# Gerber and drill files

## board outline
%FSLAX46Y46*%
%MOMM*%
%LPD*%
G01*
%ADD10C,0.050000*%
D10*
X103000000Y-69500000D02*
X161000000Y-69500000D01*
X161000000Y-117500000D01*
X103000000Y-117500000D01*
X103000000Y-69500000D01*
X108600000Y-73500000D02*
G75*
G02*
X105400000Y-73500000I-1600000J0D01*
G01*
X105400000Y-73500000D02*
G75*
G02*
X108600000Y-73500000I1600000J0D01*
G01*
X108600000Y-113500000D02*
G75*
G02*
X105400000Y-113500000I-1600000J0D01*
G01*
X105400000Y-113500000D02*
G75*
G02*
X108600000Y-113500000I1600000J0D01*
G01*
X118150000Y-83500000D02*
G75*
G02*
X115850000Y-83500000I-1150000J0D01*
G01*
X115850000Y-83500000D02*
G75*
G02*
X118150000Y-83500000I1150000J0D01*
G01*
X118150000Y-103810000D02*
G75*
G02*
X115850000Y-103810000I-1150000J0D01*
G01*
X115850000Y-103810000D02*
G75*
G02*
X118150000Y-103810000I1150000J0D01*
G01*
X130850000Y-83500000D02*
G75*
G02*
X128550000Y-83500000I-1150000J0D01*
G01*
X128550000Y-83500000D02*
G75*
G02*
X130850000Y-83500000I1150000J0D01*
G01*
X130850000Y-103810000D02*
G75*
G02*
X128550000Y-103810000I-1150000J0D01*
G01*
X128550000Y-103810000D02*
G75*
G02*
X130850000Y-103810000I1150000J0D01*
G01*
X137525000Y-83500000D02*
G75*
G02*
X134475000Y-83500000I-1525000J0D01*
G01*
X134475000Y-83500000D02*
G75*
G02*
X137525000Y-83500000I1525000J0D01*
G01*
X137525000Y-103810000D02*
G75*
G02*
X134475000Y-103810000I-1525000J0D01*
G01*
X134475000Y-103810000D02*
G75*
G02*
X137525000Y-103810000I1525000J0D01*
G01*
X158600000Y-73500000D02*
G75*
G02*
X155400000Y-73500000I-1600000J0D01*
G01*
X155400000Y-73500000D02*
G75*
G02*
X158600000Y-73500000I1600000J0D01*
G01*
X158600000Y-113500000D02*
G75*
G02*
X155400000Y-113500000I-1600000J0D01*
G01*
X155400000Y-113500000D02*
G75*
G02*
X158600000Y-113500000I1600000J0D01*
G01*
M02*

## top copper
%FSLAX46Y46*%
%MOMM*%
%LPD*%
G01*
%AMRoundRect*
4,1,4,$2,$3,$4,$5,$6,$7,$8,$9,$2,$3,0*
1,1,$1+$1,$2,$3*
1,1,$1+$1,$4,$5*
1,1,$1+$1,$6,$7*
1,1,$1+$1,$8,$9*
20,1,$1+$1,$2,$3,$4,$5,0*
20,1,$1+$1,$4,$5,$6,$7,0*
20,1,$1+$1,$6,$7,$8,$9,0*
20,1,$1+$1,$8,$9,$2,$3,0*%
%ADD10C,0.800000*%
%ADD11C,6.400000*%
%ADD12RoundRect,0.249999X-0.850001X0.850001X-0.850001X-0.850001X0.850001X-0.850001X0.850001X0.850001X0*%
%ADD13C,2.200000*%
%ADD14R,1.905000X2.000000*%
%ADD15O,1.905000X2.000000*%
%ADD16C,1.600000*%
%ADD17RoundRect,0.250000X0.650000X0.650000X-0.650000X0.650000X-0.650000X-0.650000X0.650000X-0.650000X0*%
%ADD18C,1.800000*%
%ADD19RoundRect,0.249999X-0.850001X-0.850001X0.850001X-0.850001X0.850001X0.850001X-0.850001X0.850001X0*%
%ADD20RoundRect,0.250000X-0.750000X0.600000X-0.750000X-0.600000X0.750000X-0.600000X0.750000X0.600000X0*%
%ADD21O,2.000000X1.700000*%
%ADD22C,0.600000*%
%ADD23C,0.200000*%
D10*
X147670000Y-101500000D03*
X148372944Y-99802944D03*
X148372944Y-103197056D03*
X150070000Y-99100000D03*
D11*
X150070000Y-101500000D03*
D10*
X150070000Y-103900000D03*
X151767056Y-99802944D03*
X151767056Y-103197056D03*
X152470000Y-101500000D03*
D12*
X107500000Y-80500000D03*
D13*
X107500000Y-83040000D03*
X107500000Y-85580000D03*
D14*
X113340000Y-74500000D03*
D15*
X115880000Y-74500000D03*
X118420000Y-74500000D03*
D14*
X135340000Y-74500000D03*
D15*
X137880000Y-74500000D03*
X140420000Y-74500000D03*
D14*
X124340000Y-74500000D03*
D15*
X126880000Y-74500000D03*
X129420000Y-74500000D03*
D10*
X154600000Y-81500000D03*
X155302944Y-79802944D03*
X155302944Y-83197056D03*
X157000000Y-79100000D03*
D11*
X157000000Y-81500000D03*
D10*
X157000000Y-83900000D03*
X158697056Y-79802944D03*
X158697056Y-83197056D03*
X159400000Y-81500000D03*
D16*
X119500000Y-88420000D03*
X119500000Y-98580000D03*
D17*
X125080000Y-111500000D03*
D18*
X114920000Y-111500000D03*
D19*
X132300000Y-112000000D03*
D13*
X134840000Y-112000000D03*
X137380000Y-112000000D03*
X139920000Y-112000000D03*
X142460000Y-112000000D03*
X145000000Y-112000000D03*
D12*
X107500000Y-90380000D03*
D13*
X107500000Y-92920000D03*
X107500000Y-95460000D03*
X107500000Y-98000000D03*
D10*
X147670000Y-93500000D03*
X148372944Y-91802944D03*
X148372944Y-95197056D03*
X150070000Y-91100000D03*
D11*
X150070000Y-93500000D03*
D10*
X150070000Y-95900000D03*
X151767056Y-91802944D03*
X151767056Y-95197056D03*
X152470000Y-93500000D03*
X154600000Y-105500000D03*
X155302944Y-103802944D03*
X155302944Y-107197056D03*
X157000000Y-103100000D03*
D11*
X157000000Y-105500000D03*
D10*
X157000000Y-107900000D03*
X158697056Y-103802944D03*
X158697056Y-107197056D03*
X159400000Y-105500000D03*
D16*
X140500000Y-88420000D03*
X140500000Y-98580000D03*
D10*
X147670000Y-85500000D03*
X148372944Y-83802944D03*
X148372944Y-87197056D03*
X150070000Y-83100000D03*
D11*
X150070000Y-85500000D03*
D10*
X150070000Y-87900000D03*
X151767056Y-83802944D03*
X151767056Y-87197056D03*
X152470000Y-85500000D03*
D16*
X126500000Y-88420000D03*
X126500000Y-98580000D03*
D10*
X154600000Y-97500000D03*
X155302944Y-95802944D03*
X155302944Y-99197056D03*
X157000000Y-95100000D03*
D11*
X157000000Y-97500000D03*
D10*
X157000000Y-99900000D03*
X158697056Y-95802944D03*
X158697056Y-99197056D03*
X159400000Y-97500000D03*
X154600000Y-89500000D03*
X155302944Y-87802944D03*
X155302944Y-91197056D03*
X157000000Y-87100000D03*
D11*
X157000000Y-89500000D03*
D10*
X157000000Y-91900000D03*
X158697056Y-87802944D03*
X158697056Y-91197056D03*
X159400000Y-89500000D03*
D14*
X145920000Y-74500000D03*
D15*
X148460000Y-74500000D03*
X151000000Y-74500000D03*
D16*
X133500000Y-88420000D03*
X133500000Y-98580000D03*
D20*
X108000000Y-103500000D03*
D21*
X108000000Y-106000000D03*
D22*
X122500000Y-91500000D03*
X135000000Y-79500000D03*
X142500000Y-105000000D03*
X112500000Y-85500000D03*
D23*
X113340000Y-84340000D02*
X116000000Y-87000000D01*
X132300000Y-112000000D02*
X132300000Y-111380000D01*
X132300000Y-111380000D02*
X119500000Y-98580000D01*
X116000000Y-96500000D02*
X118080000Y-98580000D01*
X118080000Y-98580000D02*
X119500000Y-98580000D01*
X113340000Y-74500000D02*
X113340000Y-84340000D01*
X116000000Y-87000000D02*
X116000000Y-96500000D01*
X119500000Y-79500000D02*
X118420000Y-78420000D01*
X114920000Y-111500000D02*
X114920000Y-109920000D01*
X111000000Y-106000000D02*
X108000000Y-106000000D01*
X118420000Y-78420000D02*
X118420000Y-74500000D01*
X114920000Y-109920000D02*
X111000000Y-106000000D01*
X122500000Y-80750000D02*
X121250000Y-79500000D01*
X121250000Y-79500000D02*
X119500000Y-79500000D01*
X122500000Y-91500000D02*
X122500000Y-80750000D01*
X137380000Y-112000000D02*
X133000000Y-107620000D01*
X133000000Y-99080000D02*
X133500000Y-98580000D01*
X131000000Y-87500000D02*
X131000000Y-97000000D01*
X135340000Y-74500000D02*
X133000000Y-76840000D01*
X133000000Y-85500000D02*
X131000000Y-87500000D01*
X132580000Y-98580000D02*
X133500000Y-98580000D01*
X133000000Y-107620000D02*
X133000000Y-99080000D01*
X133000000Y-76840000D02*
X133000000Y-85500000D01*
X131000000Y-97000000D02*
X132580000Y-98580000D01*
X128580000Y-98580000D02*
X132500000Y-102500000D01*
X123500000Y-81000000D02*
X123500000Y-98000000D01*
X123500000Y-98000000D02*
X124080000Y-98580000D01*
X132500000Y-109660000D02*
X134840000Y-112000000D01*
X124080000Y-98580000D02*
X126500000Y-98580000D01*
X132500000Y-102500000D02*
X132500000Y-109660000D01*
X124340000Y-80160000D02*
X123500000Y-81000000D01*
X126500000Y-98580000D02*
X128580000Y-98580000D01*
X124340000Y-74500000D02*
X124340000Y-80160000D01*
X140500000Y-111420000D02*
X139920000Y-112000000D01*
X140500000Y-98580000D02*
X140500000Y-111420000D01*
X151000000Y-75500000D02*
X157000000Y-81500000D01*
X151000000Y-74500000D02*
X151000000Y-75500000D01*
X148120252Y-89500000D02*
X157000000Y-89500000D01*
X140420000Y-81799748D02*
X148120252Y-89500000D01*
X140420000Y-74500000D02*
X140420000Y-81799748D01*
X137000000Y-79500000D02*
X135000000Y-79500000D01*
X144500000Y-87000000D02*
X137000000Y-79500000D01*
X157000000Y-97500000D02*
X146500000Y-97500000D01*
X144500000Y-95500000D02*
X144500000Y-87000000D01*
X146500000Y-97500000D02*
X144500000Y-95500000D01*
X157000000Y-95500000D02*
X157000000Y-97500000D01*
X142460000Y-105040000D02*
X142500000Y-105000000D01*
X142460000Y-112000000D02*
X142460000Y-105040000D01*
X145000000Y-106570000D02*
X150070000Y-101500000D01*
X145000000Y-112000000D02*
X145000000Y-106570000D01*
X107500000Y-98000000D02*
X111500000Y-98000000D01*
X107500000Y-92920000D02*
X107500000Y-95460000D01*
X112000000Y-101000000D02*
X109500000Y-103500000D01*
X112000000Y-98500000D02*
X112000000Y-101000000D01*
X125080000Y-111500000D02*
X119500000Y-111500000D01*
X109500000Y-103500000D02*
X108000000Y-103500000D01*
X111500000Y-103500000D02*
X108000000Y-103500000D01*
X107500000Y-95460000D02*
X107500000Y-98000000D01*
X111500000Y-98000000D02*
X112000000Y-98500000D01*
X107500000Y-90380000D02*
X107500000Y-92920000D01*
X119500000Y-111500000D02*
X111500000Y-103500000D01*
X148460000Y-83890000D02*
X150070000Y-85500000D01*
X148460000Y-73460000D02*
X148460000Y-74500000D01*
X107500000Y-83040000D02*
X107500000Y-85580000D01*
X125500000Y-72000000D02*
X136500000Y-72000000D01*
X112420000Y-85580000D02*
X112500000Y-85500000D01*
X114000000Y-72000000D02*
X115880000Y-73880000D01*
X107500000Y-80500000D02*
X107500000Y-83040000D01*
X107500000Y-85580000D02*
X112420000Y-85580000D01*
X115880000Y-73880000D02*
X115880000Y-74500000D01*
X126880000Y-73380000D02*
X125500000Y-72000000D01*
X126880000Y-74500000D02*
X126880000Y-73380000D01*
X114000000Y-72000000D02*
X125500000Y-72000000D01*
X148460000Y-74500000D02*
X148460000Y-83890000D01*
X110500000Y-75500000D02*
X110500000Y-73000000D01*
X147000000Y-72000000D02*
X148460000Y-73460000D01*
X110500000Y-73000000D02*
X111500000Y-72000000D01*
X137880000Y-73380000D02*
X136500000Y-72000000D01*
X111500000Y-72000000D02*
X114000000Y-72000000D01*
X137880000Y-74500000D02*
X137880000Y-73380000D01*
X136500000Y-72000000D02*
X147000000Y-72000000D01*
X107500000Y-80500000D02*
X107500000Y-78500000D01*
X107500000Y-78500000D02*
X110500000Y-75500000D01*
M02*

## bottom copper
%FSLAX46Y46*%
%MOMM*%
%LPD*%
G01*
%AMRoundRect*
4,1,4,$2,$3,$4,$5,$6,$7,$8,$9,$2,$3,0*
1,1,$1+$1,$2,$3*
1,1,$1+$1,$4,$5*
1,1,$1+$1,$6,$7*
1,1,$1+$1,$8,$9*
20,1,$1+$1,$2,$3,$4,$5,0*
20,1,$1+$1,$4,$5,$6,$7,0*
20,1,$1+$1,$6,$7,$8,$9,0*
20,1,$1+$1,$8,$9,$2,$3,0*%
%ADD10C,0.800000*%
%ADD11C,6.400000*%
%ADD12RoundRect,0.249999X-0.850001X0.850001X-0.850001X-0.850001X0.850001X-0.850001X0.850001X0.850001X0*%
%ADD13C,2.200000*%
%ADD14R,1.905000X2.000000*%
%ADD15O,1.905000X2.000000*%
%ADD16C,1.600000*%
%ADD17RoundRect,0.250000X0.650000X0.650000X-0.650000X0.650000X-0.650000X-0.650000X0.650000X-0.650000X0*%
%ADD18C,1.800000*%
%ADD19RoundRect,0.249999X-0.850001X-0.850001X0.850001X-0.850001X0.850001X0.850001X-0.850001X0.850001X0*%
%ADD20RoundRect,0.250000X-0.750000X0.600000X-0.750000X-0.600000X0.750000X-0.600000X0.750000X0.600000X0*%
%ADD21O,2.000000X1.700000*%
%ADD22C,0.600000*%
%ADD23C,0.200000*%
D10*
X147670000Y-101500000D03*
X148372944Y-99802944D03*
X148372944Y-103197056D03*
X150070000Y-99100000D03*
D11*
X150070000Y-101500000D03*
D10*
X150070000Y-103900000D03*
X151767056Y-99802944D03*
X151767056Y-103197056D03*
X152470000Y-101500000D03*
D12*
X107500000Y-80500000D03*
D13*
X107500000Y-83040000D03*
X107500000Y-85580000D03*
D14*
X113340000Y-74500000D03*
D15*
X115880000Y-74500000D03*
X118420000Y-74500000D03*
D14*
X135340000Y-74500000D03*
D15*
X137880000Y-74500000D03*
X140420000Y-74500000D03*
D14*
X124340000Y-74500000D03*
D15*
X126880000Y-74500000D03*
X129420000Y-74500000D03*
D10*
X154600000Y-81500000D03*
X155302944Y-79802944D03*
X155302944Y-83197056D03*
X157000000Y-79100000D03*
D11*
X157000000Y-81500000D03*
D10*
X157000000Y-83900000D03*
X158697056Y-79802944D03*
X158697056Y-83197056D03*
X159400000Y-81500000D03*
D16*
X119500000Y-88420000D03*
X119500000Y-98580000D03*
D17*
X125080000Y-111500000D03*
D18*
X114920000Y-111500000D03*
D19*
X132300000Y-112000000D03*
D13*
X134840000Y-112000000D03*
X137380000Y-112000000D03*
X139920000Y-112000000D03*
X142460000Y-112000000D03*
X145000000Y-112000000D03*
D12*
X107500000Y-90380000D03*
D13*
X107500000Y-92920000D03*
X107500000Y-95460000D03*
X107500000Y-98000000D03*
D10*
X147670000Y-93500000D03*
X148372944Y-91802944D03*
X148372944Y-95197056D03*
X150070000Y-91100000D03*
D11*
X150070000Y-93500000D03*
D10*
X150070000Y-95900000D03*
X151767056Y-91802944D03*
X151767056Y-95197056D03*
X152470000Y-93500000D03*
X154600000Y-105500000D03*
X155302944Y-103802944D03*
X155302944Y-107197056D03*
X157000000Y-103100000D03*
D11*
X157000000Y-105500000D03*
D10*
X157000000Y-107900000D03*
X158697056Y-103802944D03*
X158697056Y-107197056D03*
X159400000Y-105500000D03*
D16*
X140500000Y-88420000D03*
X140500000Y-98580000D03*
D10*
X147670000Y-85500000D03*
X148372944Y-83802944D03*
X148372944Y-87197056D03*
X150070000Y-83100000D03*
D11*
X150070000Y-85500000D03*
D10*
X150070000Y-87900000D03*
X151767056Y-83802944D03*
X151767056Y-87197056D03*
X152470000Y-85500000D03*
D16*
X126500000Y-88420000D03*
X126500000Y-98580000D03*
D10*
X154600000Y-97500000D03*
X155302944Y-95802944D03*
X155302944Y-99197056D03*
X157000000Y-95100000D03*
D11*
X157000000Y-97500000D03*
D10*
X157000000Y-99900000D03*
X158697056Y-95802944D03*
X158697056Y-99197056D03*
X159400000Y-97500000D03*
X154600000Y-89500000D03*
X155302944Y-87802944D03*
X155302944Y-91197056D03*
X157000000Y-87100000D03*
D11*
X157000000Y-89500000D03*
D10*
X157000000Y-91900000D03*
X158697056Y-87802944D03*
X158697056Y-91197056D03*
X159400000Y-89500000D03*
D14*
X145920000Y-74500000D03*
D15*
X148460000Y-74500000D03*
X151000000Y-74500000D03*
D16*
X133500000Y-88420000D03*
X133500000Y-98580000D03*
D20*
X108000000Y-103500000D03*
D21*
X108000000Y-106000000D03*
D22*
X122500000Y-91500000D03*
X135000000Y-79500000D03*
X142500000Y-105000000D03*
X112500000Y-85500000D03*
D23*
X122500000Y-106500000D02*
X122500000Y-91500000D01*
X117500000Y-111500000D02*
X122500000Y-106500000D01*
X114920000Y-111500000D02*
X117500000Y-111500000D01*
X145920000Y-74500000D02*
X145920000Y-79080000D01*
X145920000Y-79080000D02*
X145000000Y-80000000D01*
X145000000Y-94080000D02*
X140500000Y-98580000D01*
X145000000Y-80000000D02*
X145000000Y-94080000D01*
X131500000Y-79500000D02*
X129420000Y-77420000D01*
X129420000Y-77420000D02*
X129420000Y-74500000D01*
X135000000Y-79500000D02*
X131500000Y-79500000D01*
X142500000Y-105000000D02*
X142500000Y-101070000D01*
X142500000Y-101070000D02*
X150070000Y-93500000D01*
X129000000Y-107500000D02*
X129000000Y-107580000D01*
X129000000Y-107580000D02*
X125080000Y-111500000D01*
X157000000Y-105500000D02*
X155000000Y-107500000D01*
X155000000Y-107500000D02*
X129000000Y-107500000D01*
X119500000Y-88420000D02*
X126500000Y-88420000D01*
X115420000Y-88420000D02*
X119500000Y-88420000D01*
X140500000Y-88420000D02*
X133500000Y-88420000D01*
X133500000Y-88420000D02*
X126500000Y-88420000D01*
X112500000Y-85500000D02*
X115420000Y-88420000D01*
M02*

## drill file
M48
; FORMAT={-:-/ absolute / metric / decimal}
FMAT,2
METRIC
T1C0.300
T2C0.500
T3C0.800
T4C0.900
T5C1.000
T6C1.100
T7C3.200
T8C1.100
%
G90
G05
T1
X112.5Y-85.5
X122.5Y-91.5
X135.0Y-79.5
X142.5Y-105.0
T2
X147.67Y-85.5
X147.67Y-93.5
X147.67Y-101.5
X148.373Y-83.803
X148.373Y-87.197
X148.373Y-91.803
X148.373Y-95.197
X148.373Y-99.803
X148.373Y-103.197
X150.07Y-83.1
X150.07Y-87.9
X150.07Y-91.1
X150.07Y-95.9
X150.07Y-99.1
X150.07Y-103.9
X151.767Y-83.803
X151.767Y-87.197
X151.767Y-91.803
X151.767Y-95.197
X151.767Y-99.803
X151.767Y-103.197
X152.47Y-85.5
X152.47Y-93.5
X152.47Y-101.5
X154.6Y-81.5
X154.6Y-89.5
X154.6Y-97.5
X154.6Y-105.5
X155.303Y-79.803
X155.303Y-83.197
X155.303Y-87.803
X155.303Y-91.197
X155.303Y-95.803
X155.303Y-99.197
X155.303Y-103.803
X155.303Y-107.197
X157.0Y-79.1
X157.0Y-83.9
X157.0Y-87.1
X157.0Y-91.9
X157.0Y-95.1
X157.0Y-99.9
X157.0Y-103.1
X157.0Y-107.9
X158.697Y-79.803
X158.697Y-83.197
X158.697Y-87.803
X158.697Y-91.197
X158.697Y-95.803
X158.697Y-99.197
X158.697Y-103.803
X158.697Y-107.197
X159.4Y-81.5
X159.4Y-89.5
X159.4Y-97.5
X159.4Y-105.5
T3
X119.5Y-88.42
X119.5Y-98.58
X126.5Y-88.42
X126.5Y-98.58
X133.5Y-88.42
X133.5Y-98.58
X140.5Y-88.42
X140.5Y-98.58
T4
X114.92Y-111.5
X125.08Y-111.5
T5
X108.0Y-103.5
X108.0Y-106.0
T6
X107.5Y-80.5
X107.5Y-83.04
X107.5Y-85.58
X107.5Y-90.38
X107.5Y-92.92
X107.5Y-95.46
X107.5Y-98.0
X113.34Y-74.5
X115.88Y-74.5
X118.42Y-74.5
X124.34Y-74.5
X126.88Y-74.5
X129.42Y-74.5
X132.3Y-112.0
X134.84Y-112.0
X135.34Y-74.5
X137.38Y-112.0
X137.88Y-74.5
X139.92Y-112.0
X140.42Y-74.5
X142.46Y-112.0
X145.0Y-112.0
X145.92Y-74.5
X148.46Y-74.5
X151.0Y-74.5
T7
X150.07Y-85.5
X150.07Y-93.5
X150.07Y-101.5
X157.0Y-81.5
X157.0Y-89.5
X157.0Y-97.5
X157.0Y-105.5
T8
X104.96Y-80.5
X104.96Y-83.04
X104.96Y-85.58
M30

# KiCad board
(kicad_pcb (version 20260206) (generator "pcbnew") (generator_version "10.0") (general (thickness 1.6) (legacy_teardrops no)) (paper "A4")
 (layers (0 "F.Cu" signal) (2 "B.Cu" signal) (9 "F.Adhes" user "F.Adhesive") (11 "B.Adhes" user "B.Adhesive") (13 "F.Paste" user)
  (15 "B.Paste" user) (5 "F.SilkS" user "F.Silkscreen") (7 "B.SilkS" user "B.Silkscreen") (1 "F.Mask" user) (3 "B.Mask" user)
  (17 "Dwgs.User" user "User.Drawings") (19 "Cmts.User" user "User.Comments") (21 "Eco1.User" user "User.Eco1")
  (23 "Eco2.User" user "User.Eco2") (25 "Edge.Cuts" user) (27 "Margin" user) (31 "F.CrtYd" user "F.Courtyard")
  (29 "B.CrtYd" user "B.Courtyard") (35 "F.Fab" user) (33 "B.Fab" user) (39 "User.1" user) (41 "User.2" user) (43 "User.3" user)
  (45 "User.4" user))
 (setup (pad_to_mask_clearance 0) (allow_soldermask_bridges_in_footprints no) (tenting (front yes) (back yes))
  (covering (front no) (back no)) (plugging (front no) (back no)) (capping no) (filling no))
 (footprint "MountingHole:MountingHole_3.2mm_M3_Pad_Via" (layer "F.Cu") (at 150.07 101.5)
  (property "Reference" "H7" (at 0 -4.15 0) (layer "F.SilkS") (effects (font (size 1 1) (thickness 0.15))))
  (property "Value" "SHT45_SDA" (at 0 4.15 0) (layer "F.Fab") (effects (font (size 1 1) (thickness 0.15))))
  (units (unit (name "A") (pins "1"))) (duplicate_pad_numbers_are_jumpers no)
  (pad "1" thru_hole circle (at -2.4 0) (size 0.8 0.8) (drill 0.5) (layers "*.Cu" "*.Mask") (remove_unused_layers no) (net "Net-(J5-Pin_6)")
   (zone_connect 2))
  (pad "1" thru_hole circle (at -1.697056 -1.697056) (size 0.8 0.8) (drill 0.5) (layers "*.Cu" "*.Mask") (remove_unused_layers no)
   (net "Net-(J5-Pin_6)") (zone_connect 2))
  (pad "1" thru_hole circle (at -1.697056 1.697056) (size 0.8 0.8) (drill 0.5) (layers "*.Cu" "*.Mask") (remove_unused_layers no)
   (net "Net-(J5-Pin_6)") (zone_connect 2))
  (pad "1" thru_hole circle (at 0 -2.4) (size 0.8 0.8) (drill 0.5) (layers "*.Cu" "*.Mask") (remove_unused_layers no) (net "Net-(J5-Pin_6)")
   (zone_connect 2))
  (pad "1" thru_hole circle (at 0 0) (size 6.4 6.4) (drill 3.2) (layers "*.Cu" "*.Mask") (remove_unused_layers no) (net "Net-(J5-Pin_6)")
   (zone_connect 2))
  (pad "1" thru_hole circle (at 0 2.4) (size 0.8 0.8) (drill 0.5) (layers "*.Cu" "*.Mask") (remove_unused_layers no) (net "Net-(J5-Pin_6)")
   (zone_connect 2))
  (pad "1" thru_hole circle (at 1.697056 -1.697056) (size 0.8 0.8) (drill 0.5) (layers "*.Cu" "*.Mask") (remove_unused_layers no)
   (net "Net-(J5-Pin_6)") (zone_connect 2))
  (pad "1" thru_hole circle (at 1.697056 1.697056) (size 0.8 0.8) (drill 0.5) (layers "*.Cu" "*.Mask") (remove_unused_layers no)
   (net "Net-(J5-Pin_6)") (zone_connect 2))
  (pad "1" thru_hole circle (at 2.4 0) (size 0.8 0.8) (drill 0.5) (layers "*.Cu" "*.Mask") (remove_unused_layers no) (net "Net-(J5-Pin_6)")
   (zone_connect 2)))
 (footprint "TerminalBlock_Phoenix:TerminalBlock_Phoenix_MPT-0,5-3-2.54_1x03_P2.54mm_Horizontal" (layer "F.Cu") (at 107.5 80.5 -90)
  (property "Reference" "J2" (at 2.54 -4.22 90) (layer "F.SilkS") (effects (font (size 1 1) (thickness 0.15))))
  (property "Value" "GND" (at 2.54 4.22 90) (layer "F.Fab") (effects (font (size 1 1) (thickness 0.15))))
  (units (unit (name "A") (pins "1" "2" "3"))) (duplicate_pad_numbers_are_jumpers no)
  (pad "" np_thru_hole circle (at 0 2.54 270) (size 1.1 1.1) (drill 1.1) (layers "*.Cu" "*.Mask"))
  (pad "" np_thru_hole circle (at 2.54 2.54 270) (size 1.1 1.1) (drill 1.1) (layers "*.Cu" "*.Mask"))
  (pad "" np_thru_hole circle (at 5.08 2.54 270) (size 1.1 1.1) (drill 1.1) (layers "*.Cu" "*.Mask"))
  (pad "1" thru_hole roundrect (at 0 0 270) (size 2.2 2.2) (drill 1.1) (layers "*.Cu" "*.Mask") (remove_unused_layers no)
   (roundrect_rratio 0.113636) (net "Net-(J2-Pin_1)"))
  (pad "2" thru_hole circle (at 2.54 0 270) (size 2.2 2.2) (drill 1.1) (layers "*.Cu" "*.Mask") (remove_unused_layers no)
   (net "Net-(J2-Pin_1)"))
  (pad "3" thru_hole circle (at 5.08 0 270) (size 2.2 2.2) (drill 1.1) (layers "*.Cu" "*.Mask") (remove_unused_layers no)
   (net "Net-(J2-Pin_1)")))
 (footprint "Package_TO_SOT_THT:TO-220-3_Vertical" (layer "F.Cu") (at 113.34 74.5)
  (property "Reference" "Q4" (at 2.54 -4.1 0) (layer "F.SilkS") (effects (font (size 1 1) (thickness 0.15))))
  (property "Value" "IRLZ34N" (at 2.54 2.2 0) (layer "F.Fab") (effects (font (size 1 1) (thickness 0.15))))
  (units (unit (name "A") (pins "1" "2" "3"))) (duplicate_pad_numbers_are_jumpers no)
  (pad "1" thru_hole rect (at 0 0) (size 1.905 2) (drill 1.1) (layers "*.Cu" "*.Mask") (remove_unused_layers no) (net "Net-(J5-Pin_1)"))
  (pad "2" thru_hole oval (at 2.54 0) (size 1.905 2) (drill 1.1) (layers "*.Cu" "*.Mask") (remove_unused_layers no) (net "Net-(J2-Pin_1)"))
  (pad "3" thru_hole oval (at 5.08 0) (size 1.905 2) (drill 1.1) (layers "*.Cu" "*.Mask") (remove_unused_layers no) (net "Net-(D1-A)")))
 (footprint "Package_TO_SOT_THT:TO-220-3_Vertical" (layer "F.Cu") (at 135.34 74.5)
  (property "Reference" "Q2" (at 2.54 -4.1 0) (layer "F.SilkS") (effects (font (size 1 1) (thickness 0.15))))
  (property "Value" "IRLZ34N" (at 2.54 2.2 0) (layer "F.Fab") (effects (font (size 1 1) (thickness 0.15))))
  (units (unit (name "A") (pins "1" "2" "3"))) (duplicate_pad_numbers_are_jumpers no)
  (pad "1" thru_hole rect (at 0 0) (size 1.905 2) (drill 1.1) (layers "*.Cu" "*.Mask") (remove_unused_layers no) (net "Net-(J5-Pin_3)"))
  (pad "2" thru_hole oval (at 2.54 0) (size 1.905 2) (drill 1.1) (layers "*.Cu" "*.Mask") (remove_unused_layers no) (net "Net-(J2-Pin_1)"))
  (pad "3" thru_hole oval (at 5.08 0) (size 1.905 2) (drill 1.1) (layers "*.Cu" "*.Mask") (remove_unused_layers no) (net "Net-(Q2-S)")))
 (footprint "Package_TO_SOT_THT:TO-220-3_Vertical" (layer "F.Cu") (at 124.34 74.5)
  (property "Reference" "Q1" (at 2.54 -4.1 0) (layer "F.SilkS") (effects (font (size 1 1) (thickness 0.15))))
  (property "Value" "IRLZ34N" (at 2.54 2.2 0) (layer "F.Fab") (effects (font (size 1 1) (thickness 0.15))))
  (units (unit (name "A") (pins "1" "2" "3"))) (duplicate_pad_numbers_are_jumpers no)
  (pad "1" thru_hole rect (at 0 0) (size 1.905 2) (drill 1.1) (layers "*.Cu" "*.Mask") (remove_unused_layers no) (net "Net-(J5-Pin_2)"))
  (pad "2" thru_hole oval (at 2.54 0) (size 1.905 2) (drill 1.1) (layers "*.Cu" "*.Mask") (remove_unused_layers no) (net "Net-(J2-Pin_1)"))
  (pad "3" thru_hole oval (at 5.08 0) (size 1.905 2) (drill 1.1) (layers "*.Cu" "*.Mask") (remove_unused_layers no) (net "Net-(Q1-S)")))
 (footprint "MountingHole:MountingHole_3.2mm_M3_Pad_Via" (layer "F.Cu") (at 157 81.5)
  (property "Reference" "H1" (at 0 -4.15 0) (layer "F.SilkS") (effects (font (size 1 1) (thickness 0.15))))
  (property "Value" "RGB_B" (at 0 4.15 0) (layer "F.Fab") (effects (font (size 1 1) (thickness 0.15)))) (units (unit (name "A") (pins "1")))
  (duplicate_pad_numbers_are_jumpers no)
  (pad "1" thru_hole circle (at -2.4 0) (size 0.8 0.8) (drill 0.5) (layers "*.Cu" "*.Mask") (remove_unused_layers no) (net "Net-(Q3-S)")
   (zone_connect 2))
  (pad "1" thru_hole circle (at -1.697056 -1.697056) (size 0.8 0.8) (drill 0.5) (layers "*.Cu" "*.Mask") (remove_unused_layers no)
   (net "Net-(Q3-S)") (zone_connect 2))
  (pad "1" thru_hole circle (at -1.697056 1.697056) (size 0.8 0.8) (drill 0.5) (layers "*.Cu" "*.Mask") (remove_unused_layers no)
   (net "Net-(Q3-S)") (zone_connect 2))
  (pad "1" thru_hole circle (at 0 -2.4) (size 0.8 0.8) (drill 0.5) (layers "*.Cu" "*.Mask") (remove_unused_layers no) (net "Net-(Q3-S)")
   (zone_connect 2))
  (pad "1" thru_hole circle (at 0 0) (size 6.4 6.4) (drill 3.2) (layers "*.Cu" "*.Mask") (remove_unused_layers no) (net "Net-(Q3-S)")
   (zone_connect 2))
  (pad "1" thru_hole circle (at 0 2.4) (size 0.8 0.8) (drill 0.5) (layers "*.Cu" "*.Mask") (remove_unused_layers no) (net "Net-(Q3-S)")
   (zone_connect 2))
  (pad "1" thru_hole circle (at 1.697056 -1.697056) (size 0.8 0.8) (drill 0.5) (layers "*.Cu" "*.Mask") (remove_unused_layers no)
   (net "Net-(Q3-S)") (zone_connect 2))
  (pad "1" thru_hole circle (at 1.697056 1.697056) (size 0.8 0.8) (drill 0.5) (layers "*.Cu" "*.Mask") (remove_unused_layers no)
   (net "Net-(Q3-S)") (zone_connect 2))
  (pad "1" thru_hole circle (at 2.4 0) (size 0.8 0.8) (drill 0.5) (layers "*.Cu" "*.Mask") (remove_unused_layers no) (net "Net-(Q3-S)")
   (zone_connect 2)))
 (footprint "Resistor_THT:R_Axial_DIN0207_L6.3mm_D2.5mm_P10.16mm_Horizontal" (layer "F.Cu") (at 119.5 88.42 -90)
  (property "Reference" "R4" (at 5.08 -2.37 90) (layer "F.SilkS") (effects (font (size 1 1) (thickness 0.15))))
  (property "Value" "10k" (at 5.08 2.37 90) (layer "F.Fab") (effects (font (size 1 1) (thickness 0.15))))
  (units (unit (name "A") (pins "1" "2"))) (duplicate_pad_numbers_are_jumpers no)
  (pad "1" thru_hole circle (at 0 0 270) (size 1.6 1.6) (drill 0.8) (layers "*.Cu" "*.Mask") (remove_unused_layers no)
   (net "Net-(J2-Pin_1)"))
  (pad "2" thru_hole circle (at 10.16 0 270) (size 1.6 1.6) (drill 0.8) (layers "*.Cu" "*.Mask") (remove_unused_layers no)
   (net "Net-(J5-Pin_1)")))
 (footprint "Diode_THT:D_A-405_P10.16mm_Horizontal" (layer "F.Cu") (at 125.08 111.5 180)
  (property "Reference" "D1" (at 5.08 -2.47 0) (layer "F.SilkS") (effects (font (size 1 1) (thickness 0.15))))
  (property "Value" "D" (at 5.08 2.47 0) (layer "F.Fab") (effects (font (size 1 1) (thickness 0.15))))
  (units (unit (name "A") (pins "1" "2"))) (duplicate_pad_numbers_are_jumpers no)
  (pad "1" thru_hole roundrect (at 0 0 180) (size 1.8 1.8) (drill 0.9) (layers "*.Cu" "*.Mask") (remove_unused_layers no)
   (roundrect_rratio 0.138889) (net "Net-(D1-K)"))
  (pad "2" thru_hole circle (at 10.16 0 180) (size 1.8 1.8) (drill 0.9) (layers "*.Cu" "*.Mask") (remove_unused_layers no)
   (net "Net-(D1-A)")))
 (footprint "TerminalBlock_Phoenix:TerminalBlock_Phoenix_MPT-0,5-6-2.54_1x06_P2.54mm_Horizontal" (layer "F.Cu") (at 132.3 112)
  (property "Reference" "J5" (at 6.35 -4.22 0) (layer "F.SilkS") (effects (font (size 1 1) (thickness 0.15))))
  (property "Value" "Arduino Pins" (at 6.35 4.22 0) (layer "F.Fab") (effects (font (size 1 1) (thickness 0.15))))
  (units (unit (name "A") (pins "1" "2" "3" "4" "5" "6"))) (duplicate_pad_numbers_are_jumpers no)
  (pad "1" thru_hole roundrect (at 0 0) (size 2.2 2.2) (drill 1.1) (layers "*.Cu" "*.Mask") (remove_unused_layers no)
   (roundrect_rratio 0.113636) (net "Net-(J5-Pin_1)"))
  (pad "2" thru_hole circle (at 2.54 0) (size 2.2 2.2) (drill 1.1) (layers "*.Cu" "*.Mask") (remove_unused_layers no) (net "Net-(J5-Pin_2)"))
  (pad "3" thru_hole circle (at 5.08 0) (size 2.2 2.2) (drill 1.1) (layers "*.Cu" "*.Mask") (remove_unused_layers no) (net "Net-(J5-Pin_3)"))
  (pad "4" thru_hole circle (at 7.62 0) (size 2.2 2.2) (drill 1.1) (layers "*.Cu" "*.Mask") (remove_unused_layers no) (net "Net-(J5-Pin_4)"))
  (pad "5" thru_hole circle (at 10.16 0) (size 2.2 2.2) (drill 1.1) (layers "*.Cu" "*.Mask") (remove_unused_layers no)
   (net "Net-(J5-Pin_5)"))
  (pad "6" thru_hole circle (at 12.7 0) (size 2.2 2.2) (drill 1.1) (layers "*.Cu" "*.Mask") (remove_unused_layers no) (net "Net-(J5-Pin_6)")))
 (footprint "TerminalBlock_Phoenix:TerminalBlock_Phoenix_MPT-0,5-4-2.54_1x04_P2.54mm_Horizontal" (layer "F.Cu") (at 107.5 90.38 -90)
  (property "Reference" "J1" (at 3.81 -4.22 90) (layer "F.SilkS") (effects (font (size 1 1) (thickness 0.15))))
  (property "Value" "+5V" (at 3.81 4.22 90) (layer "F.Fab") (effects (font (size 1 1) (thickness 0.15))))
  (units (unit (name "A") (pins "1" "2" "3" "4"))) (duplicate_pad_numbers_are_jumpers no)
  (pad "1" thru_hole roundrect (at 0 0 270) (size 2.2 2.2) (drill 1.1) (layers "*.Cu" "*.Mask") (remove_unused_layers no)
   (roundrect_rratio 0.113636) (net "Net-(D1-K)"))
  (pad "2" thru_hole circle (at 2.54 0 270) (size 2.2 2.2) (drill 1.1) (layers "*.Cu" "*.Mask") (remove_unused_layers no) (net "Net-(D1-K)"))
  (pad "3" thru_hole circle (at 5.08 0 270) (size 2.2 2.2) (drill 1.1) (layers "*.Cu" "*.Mask") (remove_unused_layers no) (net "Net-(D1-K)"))
  (pad "4" thru_hole circle (at 7.62 0 270) (size 2.2 2.2) (drill 1.1) (layers "*.Cu" "*.Mask") (remove_unused_layers no) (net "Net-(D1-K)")))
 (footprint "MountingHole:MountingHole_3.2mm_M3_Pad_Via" (layer "F.Cu") (at 150.07 93.5)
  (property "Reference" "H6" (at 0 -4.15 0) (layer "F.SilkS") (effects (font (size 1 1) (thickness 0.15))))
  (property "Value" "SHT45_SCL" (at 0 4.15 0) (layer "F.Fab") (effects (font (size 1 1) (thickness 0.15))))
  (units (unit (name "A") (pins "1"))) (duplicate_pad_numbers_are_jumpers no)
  (pad "1" thru_hole circle (at -2.4 0) (size 0.8 0.8) (drill 0.5) (layers "*.Cu" "*.Mask") (remove_unused_layers no) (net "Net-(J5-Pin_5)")
   (zone_connect 2))
  (pad "1" thru_hole circle (at -1.697056 -1.697056) (size 0.8 0.8) (drill 0.5) (layers "*.Cu" "*.Mask") (remove_unused_layers no)
   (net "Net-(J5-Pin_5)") (zone_connect 2))
  (pad "1" thru_hole circle (at -1.697056 1.697056) (size 0.8 0.8) (drill 0.5) (layers "*.Cu" "*.Mask") (remove_unused_layers no)
   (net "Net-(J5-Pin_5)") (zone_connect 2))
  (pad "1" thru_hole circle (at 0 -2.4) (size 0.8 0.8) (drill 0.5) (layers "*.Cu" "*.Mask") (remove_unused_layers no) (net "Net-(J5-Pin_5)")
   (zone_connect 2))
  (pad "1" thru_hole circle (at 0 0) (size 6.4 6.4) (drill 3.2) (layers "*.Cu" "*.Mask") (remove_unused_layers no) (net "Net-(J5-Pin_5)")
   (zone_connect 2))
  (pad "1" thru_hole circle (at 0 2.4) (size 0.8 0.8) (drill 0.5) (layers "*.Cu" "*.Mask") (remove_unused_layers no) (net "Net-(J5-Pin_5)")
   (zone_connect 2))
  (pad "1" thru_hole circle (at 1.697056 -1.697056) (size 0.8 0.8) (drill 0.5) (layers "*.Cu" "*.Mask") (remove_unused_layers no)
   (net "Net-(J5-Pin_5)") (zone_connect 2))
  (pad "1" thru_hole circle (at 1.697056 1.697056) (size 0.8 0.8) (drill 0.5) (layers "*.Cu" "*.Mask") (remove_unused_layers no)
   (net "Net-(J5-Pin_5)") (zone_connect 2))
  (pad "1" thru_hole circle (at 2.4 0) (size 0.8 0.8) (drill 0.5) (layers "*.Cu" "*.Mask") (remove_unused_layers no) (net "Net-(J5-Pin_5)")
   (zone_connect 2)))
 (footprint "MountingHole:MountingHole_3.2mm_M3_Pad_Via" (layer "F.Cu") (at 157 105.5)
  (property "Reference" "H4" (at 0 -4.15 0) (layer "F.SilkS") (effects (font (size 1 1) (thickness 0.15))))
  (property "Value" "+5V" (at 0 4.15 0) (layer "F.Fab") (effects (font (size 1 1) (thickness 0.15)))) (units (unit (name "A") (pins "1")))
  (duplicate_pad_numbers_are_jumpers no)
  (pad "1" thru_hole circle (at -2.4 0) (size 0.8 0.8) (drill 0.5) (layers "*.Cu" "*.Mask") (remove_unused_layers no) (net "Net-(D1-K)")
   (zone_connect 2))
  (pad "1" thru_hole circle (at -1.697056 -1.697056) (size 0.8 0.8) (drill 0.5) (layers "*.Cu" "*.Mask") (remove_unused_layers no)
   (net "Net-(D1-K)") (zone_connect 2))
  (pad "1" thru_hole circle (at -1.697056 1.697056) (size 0.8 0.8) (drill 0.5) (layers "*.Cu" "*.Mask") (remove_unused_layers no)
   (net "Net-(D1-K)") (zone_connect 2))
  (pad "1" thru_hole circle (at 0 -2.4) (size 0.8 0.8) (drill 0.5) (layers "*.Cu" "*.Mask") (remove_unused_layers no) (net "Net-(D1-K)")
   (zone_connect 2))
  (pad "1" thru_hole circle (at 0 0) (size 6.4 6.4) (drill 3.2) (layers "*.Cu" "*.Mask") (remove_unused_layers no) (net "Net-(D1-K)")
   (zone_connect 2))
  (pad "1" thru_hole circle (at 0 2.4) (size 0.8 0.8) (drill 0.5) (layers "*.Cu" "*.Mask") (remove_unused_layers no) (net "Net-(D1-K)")
   (zone_connect 2))
  (pad "1" thru_hole circle (at 1.697056 -1.697056) (size 0.8 0.8) (drill 0.5) (layers "*.Cu" "*.Mask") (remove_unused_layers no)
   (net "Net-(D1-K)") (zone_connect 2))
  (pad "1" thru_hole circle (at 1.697056 1.697056) (size 0.8 0.8) (drill 0.5) (layers "*.Cu" "*.Mask") (remove_unused_layers no)
   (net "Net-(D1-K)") (zone_connect 2))
  (pad "1" thru_hole circle (at 2.4 0) (size 0.8 0.8) (drill 0.5) (layers "*.Cu" "*.Mask") (remove_unused_layers no) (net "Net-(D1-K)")
   (zone_connect 2)))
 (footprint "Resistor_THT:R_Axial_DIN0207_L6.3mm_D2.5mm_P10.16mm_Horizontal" (layer "F.Cu") (at 140.5 88.42 -90)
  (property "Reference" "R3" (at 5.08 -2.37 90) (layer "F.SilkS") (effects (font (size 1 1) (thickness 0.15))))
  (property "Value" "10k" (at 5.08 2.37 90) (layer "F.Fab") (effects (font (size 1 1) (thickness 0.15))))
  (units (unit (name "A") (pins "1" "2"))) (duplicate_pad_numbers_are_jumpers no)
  (pad "1" thru_hole circle (at 0 0 270) (size 1.6 1.6) (drill 0.8) (layers "*.Cu" "*.Mask") (remove_unused_layers no)
   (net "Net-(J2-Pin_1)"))
  (pad "2" thru_hole circle (at 10.16 0 270) (size 1.6 1.6) (drill 0.8) (layers "*.Cu" "*.Mask") (remove_unused_layers no)
   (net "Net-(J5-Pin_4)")))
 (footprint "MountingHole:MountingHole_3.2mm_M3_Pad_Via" (layer "F.Cu") (at 150.07 85.5)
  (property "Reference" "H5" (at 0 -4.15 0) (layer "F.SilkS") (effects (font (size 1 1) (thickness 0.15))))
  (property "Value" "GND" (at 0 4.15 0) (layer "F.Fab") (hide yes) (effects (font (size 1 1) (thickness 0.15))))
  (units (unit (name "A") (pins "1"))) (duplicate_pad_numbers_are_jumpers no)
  (pad "1" thru_hole circle (at -2.4 0) (size 0.8 0.8) (drill 0.5) (layers "*.Cu" "*.Mask") (remove_unused_layers no) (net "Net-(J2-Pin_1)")
   (zone_connect 2))
  (pad "1" thru_hole circle (at -1.697056 -1.697056) (size 0.8 0.8) (drill 0.5) (layers "*.Cu" "*.Mask") (remove_unused_layers no)
   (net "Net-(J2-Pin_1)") (zone_connect 2))
  (pad "1" thru_hole circle (at -1.697056 1.697056) (size 0.8 0.8) (drill 0.5) (layers "*.Cu" "*.Mask") (remove_unused_layers no)
   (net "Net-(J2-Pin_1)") (zone_connect 2))
  (pad "1" thru_hole circle (at 0 -2.4) (size 0.8 0.8) (drill 0.5) (layers "*.Cu" "*.Mask") (remove_unused_layers no) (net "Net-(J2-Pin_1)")
   (zone_connect 2))
  (pad "1" thru_hole circle (at 0 0) (size 6.4 6.4) (drill 3.2) (layers "*.Cu" "*.Mask") (remove_unused_layers no) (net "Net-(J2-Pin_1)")
   (zone_connect 2))
  (pad "1" thru_hole circle (at 0 2.4) (size 0.8 0.8) (drill 0.5) (layers "*.Cu" "*.Mask") (remove_unused_layers no) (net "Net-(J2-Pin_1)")
   (zone_connect 2))
  (pad "1" thru_hole circle (at 1.697056 -1.697056) (size 0.8 0.8) (drill 0.5) (layers "*.Cu" "*.Mask") (remove_unused_layers no)
   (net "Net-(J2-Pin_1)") (zone_connect 2))
  (pad "1" thru_hole circle (at 1.697056 1.697056) (size 0.8 0.8) (drill 0.5) (layers "*.Cu" "*.Mask") (remove_unused_layers no)
   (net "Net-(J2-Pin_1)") (zone_connect 2))
  (pad "1" thru_hole circle (at 2.4 0) (size 0.8 0.8) (drill 0.5) (layers "*.Cu" "*.Mask") (remove_unused_layers no) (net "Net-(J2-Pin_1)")
   (zone_connect 2)))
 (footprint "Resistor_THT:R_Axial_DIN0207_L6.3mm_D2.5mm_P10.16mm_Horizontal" (layer "F.Cu") (at 126.5 88.42 -90)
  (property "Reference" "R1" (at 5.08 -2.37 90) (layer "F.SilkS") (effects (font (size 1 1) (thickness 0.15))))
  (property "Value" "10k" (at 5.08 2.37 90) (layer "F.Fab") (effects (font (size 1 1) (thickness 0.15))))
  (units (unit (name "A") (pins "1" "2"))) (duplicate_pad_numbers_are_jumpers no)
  (pad "1" thru_hole circle (at 0 0 270) (size 1.6 1.6) (drill 0.8) (layers "*.Cu" "*.Mask") (remove_unused_layers no)
   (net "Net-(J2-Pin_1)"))
  (pad "2" thru_hole circle (at 10.16 0 270) (size 1.6 1.6) (drill 0.8) (layers "*.Cu" "*.Mask") (remove_unused_layers no)
   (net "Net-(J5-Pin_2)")))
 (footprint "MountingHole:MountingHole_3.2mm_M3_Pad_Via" (layer "F.Cu") (at 157 97.5)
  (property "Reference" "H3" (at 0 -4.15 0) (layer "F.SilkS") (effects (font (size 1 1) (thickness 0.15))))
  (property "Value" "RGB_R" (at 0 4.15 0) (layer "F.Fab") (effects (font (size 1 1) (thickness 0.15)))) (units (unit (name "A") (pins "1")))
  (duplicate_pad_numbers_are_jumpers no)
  (pad "1" thru_hole circle (at -2.4 0) (size 0.8 0.8) (drill 0.5) (layers "*.Cu" "*.Mask") (remove_unused_layers no) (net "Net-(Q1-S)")
   (zone_connect 2))
  (pad "1" thru_hole circle (at -1.697056 -1.697056) (size 0.8 0.8) (drill 0.5) (layers "*.Cu" "*.Mask") (remove_unused_layers no)
   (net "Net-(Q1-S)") (zone_connect 2))
  (pad "1" thru_hole circle (at -1.697056 1.697056) (size 0.8 0.8) (drill 0.5) (layers "*.Cu" "*.Mask") (remove_unused_layers no)
   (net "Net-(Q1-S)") (zone_connect 2))
  (pad "1" thru_hole circle (at 0 -2.4) (size 0.8 0.8) (drill 0.5) (layers "*.Cu" "*.Mask") (remove_unused_layers no) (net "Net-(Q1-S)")
   (zone_connect 2))
  (pad "1" thru_hole circle (at 0 0) (size 6.4 6.4) (drill 3.2) (layers "*.Cu" "*.Mask") (remove_unused_layers no) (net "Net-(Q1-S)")
   (zone_connect 2))
  (pad "1" thru_hole circle (at 0 2.4) (size 0.8 0.8) (drill 0.5) (layers "*.Cu" "*.Mask") (remove_unused_layers no) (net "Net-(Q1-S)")
   (zone_connect 2))
  (pad "1" thru_hole circle (at 1.697056 -1.697056) (size 0.8 0.8) (drill 0.5) (layers "*.Cu" "*.Mask") (remove_unused_layers no)
   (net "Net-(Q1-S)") (zone_connect 2))
  (pad "1" thru_hole circle (at 1.697056 1.697056) (size 0.8 0.8) (drill 0.5) (layers "*.Cu" "*.Mask") (remove_unused_layers no)
   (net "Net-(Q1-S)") (zone_connect 2))
  (pad "1" thru_hole circle (at 2.4 0) (size 0.8 0.8) (drill 0.5) (layers "*.Cu" "*.Mask") (remove_unused_layers no) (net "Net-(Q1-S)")
   (zone_connect 2)))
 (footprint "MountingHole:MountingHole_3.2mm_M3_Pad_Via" (layer "F.Cu") (at 157 89.5)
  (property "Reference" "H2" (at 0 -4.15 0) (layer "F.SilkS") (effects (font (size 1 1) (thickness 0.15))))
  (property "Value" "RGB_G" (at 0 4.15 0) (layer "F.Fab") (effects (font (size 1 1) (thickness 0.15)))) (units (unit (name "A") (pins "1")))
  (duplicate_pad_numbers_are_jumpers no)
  (pad "1" thru_hole circle (at -2.4 0) (size 0.8 0.8) (drill 0.5) (layers "*.Cu" "*.Mask") (remove_unused_layers no) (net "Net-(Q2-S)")
   (zone_connect 2))
  (pad "1" thru_hole circle (at -1.697056 -1.697056) (size 0.8 0.8) (drill 0.5) (layers "*.Cu" "*.Mask") (remove_unused_layers no)
   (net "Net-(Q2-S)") (zone_connect 2))
  (pad "1" thru_hole circle (at -1.697056 1.697056) (size 0.8 0.8) (drill 0.5) (layers "*.Cu" "*.Mask") (remove_unused_layers no)
   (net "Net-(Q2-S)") (zone_connect 2))
  (pad "1" thru_hole circle (at 0 -2.4) (size 0.8 0.8) (drill 0.5) (layers "*.Cu" "*.Mask") (remove_unused_layers no) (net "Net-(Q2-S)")
   (zone_connect 2))
  (pad "1" thru_hole circle (at 0 0) (size 6.4 6.4) (drill 3.2) (layers "*.Cu" "*.Mask") (remove_unused_layers no) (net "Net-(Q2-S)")
   (zone_connect 2))
  (pad "1" thru_hole circle (at 0 2.4) (size 0.8 0.8) (drill 0.5) (layers "*.Cu" "*.Mask") (remove_unused_layers no) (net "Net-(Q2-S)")
   (zone_connect 2))
  (pad "1" thru_hole circle (at 1.697056 -1.697056) (size 0.8 0.8) (drill 0.5) (layers "*.Cu" "*.Mask") (remove_unused_layers no)
   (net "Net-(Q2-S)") (zone_connect 2))
  (pad "1" thru_hole circle (at 1.697056 1.697056) (size 0.8 0.8) (drill 0.5) (layers "*.Cu" "*.Mask") (remove_unused_layers no)
   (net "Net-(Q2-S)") (zone_connect 2))
  (pad "1" thru_hole circle (at 2.4 0) (size 0.8 0.8) (drill 0.5) (layers "*.Cu" "*.Mask") (remove_unused_layers no) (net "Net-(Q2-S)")
   (zone_connect 2)))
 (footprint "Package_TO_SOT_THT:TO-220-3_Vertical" (layer "F.Cu") (at 145.92 74.5)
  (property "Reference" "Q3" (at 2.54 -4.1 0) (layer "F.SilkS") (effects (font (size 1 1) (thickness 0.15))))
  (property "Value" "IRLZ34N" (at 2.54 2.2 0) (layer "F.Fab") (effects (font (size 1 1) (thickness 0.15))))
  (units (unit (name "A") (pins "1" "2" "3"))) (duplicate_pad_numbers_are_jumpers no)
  (pad "1" thru_hole rect (at 0 0) (size 1.905 2) (drill 1.1) (layers "*.Cu" "*.Mask") (remove_unused_layers no) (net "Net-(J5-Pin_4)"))
  (pad "2" thru_hole oval (at 2.54 0) (size 1.905 2) (drill 1.1) (layers "*.Cu" "*.Mask") (remove_unused_layers no) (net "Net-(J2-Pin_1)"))
  (pad "3" thru_hole oval (at 5.08 0) (size 1.905 2) (drill 1.1) (layers "*.Cu" "*.Mask") (remove_unused_layers no) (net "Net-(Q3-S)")))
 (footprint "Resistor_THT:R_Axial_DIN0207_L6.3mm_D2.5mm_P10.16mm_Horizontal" (layer "F.Cu") (at 133.5 88.42 -90)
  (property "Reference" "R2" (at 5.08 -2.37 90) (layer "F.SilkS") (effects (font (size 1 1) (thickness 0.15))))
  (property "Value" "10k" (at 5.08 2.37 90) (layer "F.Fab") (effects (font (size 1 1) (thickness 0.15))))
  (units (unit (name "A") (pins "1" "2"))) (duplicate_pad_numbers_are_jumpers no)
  (pad "1" thru_hole circle (at 0 0 270) (size 1.6 1.6) (drill 0.8) (layers "*.Cu" "*.Mask") (remove_unused_layers no)
   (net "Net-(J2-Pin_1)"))
  (pad "2" thru_hole circle (at 10.16 0 270) (size 1.6 1.6) (drill 0.8) (layers "*.Cu" "*.Mask") (remove_unused_layers no)
   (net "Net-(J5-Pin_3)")))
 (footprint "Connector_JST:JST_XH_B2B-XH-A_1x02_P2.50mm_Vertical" (layer "F.Cu") (at 108 103.5 -90)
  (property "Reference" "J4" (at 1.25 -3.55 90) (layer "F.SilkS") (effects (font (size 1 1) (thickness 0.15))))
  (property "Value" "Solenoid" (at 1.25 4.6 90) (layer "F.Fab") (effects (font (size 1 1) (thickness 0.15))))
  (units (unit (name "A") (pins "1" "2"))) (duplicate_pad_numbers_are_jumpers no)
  (pad "1" thru_hole roundrect (at 0 0 270) (size 1.7 2) (drill 1) (layers "*.Cu" "*.Mask") (remove_unused_layers no)
   (roundrect_rratio 0.147059) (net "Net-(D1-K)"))
  (pad "2" thru_hole oval (at 2.5 0 270) (size 1.7 2) (drill 1) (layers "*.Cu" "*.Mask") (remove_unused_layers no) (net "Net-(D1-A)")))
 (gr_rect (start 103 69.5) (end 161 117.5) (stroke (width 0.05) (type default)) (fill no) (layer "Edge.Cuts"))
 (gr_circle (center 107 73.5) (end 108.6 73.5) (stroke (width 0.05) (type default)) (fill no) (layer "Edge.Cuts"))
 (gr_circle (center 107 113.5) (end 108.6 113.5) (stroke (width 0.05) (type default)) (fill no) (layer "Edge.Cuts"))
 (gr_circle (center 117 83.5) (end 118.15 83.5) (stroke (width 0.05) (type default)) (fill no) (layer "Edge.Cuts"))
 (gr_circle (center 117 103.81) (end 118.15 103.81) (stroke (width 0.05) (type default)) (fill no) (layer "Edge.Cuts"))
 (gr_circle (center 129.7 83.5) (end 130.85 83.5) (stroke (width 0.05) (type default)) (fill no) (layer "Edge.Cuts"))
 (gr_circle (center 129.7 103.81) (end 130.85 103.81) (stroke (width 0.05) (type default)) (fill no) (layer "Edge.Cuts"))
 (gr_circle (center 136 83.5) (end 137.525 83.5) (stroke (width 0.05) (type default)) (fill no) (layer "Edge.Cuts"))
 (gr_circle (center 136 103.81) (end 137.525 103.81) (stroke (width 0.05) (type default)) (fill no) (layer "Edge.Cuts"))
 (gr_circle (center 157 73.5) (end 158.6 73.5) (stroke (width 0.05) (type default)) (fill no) (layer "Edge.Cuts"))
 (gr_circle (center 157 113.5) (end 158.6 113.5) (stroke (width 0.05) (type default)) (fill no) (layer "Edge.Cuts"))
 (segment (start 113.34 84.34) (end 116 87) (width 0.2) (layer "F.Cu") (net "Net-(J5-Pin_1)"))
 (segment (start 132.3 112) (end 132.3 111.38) (width 0.2) (layer "F.Cu") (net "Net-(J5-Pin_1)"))
 (segment (start 132.3 111.38) (end 119.5 98.58) (width 0.2) (layer "F.Cu") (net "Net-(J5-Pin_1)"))
 (segment (start 116 96.5) (end 118.08 98.58) (width 0.2) (layer "F.Cu") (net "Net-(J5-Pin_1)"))
 (segment (start 118.08 98.58) (end 119.5 98.58) (width 0.2) (layer "F.Cu") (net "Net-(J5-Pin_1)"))
 (segment (start 113.34 74.5) (end 113.34 84.34) (width 0.2) (layer "F.Cu") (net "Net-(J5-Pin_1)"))
 (segment (start 116 87) (end 116 96.5) (width 0.2) (layer "F.Cu") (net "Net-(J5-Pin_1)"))
 (segment (start 119.5 79.5) (end 118.42 78.42) (width 0.2) (layer "F.Cu") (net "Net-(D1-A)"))
 (segment (start 114.92 111.5) (end 114.92 109.92) (width 0.2) (layer "F.Cu") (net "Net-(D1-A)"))
 (segment (start 111 106) (end 108 106) (width 0.2) (layer "F.Cu") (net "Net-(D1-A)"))
 (segment (start 118.42 78.42) (end 118.42 74.5) (width 0.2) (layer "F.Cu") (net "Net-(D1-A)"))
 (segment (start 114.92 109.92) (end 111 106) (width 0.2) (layer "F.Cu") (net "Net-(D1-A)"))
 (segment (start 122.5 80.75) (end 121.25 79.5) (width 0.2) (layer "F.Cu") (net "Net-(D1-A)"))
 (segment (start 121.25 79.5) (end 119.5 79.5) (width 0.2) (layer "F.Cu") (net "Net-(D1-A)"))
 (segment (start 122.5 91.5) (end 122.5 80.75) (width 0.2) (layer "F.Cu") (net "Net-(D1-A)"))
 (via (at 122.5 91.5) (size 0.6) (drill 0.3) (layers "F.Cu" "B.Cu") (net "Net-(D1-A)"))
 (segment (start 122.5 106.5) (end 122.5 91.5) (width 0.2) (layer "B.Cu") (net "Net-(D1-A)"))
 (segment (start 117.5 111.5) (end 122.5 106.5) (width 0.2) (layer "B.Cu") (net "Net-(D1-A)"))
 (segment (start 114.92 111.5) (end 117.5 111.5) (width 0.2) (layer "B.Cu") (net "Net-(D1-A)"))
 (segment (start 137.38 112) (end 133 107.62) (width 0.2) (layer "F.Cu") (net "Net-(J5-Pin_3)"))
 (segment (start 133 99.08) (end 133.5 98.58) (width 0.2) (layer "F.Cu") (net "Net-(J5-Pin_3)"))
 (segment (start 131 87.5) (end 131 97) (width 0.2) (layer "F.Cu") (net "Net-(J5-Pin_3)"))
 (segment (start 135.34 74.5) (end 133 76.84) (width 0.2) (layer "F.Cu") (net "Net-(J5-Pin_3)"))
 (segment (start 133 85.5) (end 131 87.5) (width 0.2) (layer "F.Cu") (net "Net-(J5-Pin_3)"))
 (segment (start 132.58 98.58) (end 133.5 98.58) (width 0.2) (layer "F.Cu") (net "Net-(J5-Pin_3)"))
 (segment (start 133 107.62) (end 133 99.08) (width 0.2) (layer "F.Cu") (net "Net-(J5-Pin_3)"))
 (segment (start 133 76.84) (end 133 85.5) (width 0.2) (layer "F.Cu") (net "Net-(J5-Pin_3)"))
 (segment (start 131 97) (end 132.58 98.58) (width 0.2) (layer "F.Cu") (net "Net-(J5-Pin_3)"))
 (segment (start 128.58 98.58) (end 132.5 102.5) (width 0.2) (layer "F.Cu") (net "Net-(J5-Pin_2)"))
 (segment (start 123.5 81) (end 123.5 98) (width 0.2) (layer "F.Cu") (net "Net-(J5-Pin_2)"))
 (segment (start 123.5 98) (end 124.08 98.58) (width 0.2) (layer "F.Cu") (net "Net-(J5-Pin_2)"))
 (segment (start 132.5 109.66) (end 134.84 112) (width 0.2) (layer "F.Cu") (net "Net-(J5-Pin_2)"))
 (segment (start 124.08 98.58) (end 126.5 98.58) (width 0.2) (layer "F.Cu") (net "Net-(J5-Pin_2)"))
 (segment (start 132.5 102.5) (end 132.5 109.66) (width 0.2) (layer "F.Cu") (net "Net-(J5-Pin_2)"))
 (segment (start 124.34 80.16) (end 123.5 81) (width 0.2) (layer "F.Cu") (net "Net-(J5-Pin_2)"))
 (segment (start 126.5 98.58) (end 128.58 98.58) (width 0.2) (layer "F.Cu") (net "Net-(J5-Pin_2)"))
 (segment (start 124.34 74.5) (end 124.34 80.16) (width 0.2) (layer "F.Cu") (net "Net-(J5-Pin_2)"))
 (segment (start 140.5 111.42) (end 139.92 112) (width 0.2) (layer "F.Cu") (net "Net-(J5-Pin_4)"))
 (segment (start 140.5 98.58) (end 140.5 111.42) (width 0.2) (layer "F.Cu") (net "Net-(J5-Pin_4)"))
 (segment (start 145.92 74.5) (end 145.92 79.08) (width 0.2) (layer "B.Cu") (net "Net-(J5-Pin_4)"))
 (segment (start 145.92 79.08) (end 145 80) (width 0.2) (layer "B.Cu") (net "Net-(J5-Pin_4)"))
 (segment (start 145 94.08) (end 140.5 98.58) (width 0.2) (layer "B.Cu") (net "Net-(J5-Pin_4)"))
 (segment (start 145 80) (end 145 94.08) (width 0.2) (layer "B.Cu") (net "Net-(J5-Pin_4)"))
 (segment (start 151 75.5) (end 157 81.5) (width 0.2) (layer "F.Cu") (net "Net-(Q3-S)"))
 (segment (start 151 74.5) (end 151 75.5) (width 0.2) (layer "F.Cu") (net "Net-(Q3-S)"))
 (segment (start 148.120252 89.5) (end 157 89.5) (width 0.2) (layer "F.Cu") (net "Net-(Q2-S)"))
 (segment (start 140.42 81.799748) (end 148.120252 89.5) (width 0.2) (layer "F.Cu") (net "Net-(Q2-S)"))
 (segment (start 140.42 74.5) (end 140.42 81.799748) (width 0.2) (layer "F.Cu") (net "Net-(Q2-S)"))
 (segment (start 137 79.5) (end 135 79.5) (width 0.2) (layer "F.Cu") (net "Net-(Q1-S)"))
 (segment (start 144.5 87) (end 137 79.5) (width 0.2) (layer "F.Cu") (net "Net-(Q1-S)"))
 (segment (start 157 97.5) (end 146.5 97.5) (width 0.2) (layer "F.Cu") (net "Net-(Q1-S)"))
 (segment (start 144.5 95.5) (end 144.5 87) (width 0.2) (layer "F.Cu") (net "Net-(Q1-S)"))
 (segment (start 146.5 97.5) (end 144.5 95.5) (width 0.2) (layer "F.Cu") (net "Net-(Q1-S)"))
 (segment (start 157 95.5) (end 157 97.5) (width 0.2) (layer "F.Cu") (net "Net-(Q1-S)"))
 (via (at 135 79.5) (size 0.6) (drill 0.3) (layers "F.Cu" "B.Cu") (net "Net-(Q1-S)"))
 (segment (start 131.5 79.5) (end 129.42 77.42) (width 0.2) (layer "B.Cu") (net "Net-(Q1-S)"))
 (segment (start 129.42 77.42) (end 129.42 74.5) (width 0.2) (layer "B.Cu") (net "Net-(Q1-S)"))
 (segment (start 135 79.5) (end 131.5 79.5) (width 0.2) (layer "B.Cu") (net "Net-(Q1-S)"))
 (segment (start 142.46 105.04) (end 142.5 105) (width 0.2) (layer "F.Cu") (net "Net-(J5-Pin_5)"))
 (segment (start 142.46 112) (end 142.46 105.04) (width 0.2) (layer "F.Cu") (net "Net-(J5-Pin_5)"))
 (via (at 142.5 105) (size 0.6) (drill 0.3) (layers "F.Cu" "B.Cu") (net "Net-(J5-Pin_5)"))
 (segment (start 142.5 105) (end 142.5 101.07) (width 0.2) (layer "B.Cu") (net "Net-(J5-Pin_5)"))
 (segment (start 142.5 101.07) (end 150.07 93.5) (width 0.2) (layer "B.Cu") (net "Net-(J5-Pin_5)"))
 (segment (start 145 106.57) (end 150.07 101.5) (width 0.2) (layer "F.Cu") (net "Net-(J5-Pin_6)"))
 (segment (start 145 112) (end 145 106.57) (width 0.2) (layer "F.Cu") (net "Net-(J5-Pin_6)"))
 (segment (start 107.5 98) (end 111.5 98) (width 0.2) (layer "F.Cu") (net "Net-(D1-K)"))
 (segment (start 107.5 92.92) (end 107.5 95.46) (width 0.2) (layer "F.Cu") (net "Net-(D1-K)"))
 (segment (start 112 101) (end 109.5 103.5) (width 0.2) (layer "F.Cu") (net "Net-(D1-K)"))
 (segment (start 112 98.5) (end 112 101) (width 0.2) (layer "F.Cu") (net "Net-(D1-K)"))
 (segment (start 125.08 111.5) (end 119.5 111.5) (width 0.2) (layer "F.Cu") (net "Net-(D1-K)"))
 (segment (start 109.5 103.5) (end 108 103.5) (width 0.2) (layer "F.Cu") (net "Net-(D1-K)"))
 (segment (start 111.5 103.5) (end 108 103.5) (width 0.2) (layer "F.Cu") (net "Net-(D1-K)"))
 (segment (start 107.5 95.46) (end 107.5 98) (width 0.2) (layer "F.Cu") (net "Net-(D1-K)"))
 (segment (start 111.5 98) (end 112 98.5) (width 0.2) (layer "F.Cu") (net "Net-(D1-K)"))
 (segment (start 107.5 90.38) (end 107.5 92.92) (width 0.2) (layer "F.Cu") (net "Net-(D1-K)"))
 (segment (start 119.5 111.5) (end 111.5 103.5) (width 0.2) (layer "F.Cu") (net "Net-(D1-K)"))
 (segment (start 129 107.5) (end 129 107.58) (width 0.2) (layer "B.Cu") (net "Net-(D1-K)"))
 (segment (start 129 107.58) (end 125.08 111.5) (width 0.2) (layer "B.Cu") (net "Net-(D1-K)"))
 (segment (start 157 105.5) (end 155 107.5) (width 0.2) (layer "B.Cu") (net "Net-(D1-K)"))
 (segment (start 155 107.5) (end 129 107.5) (width 0.2) (layer "B.Cu") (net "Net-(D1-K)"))
 (segment (start 148.46 83.89) (end 150.07 85.5) (width 0.2) (layer "F.Cu") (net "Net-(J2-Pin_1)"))
 (segment (start 148.46 73.46) (end 148.46 74.5) (width 0.2) (layer "F.Cu") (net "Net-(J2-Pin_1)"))
 (segment (start 107.5 83.04) (end 107.5 85.58) (width 0.2) (layer "F.Cu") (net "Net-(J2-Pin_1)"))
 (segment (start 125.5 72) (end 136.5 72) (width 0.2) (layer "F.Cu") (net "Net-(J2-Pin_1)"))
 (segment (start 112.42 85.58) (end 112.5 85.5) (width 0.2) (layer "F.Cu") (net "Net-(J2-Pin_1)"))
 (segment (start 114 72) (end 115.88 73.88) (width 0.2) (layer "F.Cu") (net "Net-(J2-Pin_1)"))
 (segment (start 107.5 80.5) (end 107.5 83.04) (width 0.2) (layer "F.Cu") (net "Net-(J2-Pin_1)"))
 (segment (start 107.5 85.58) (end 112.42 85.58) (width 0.2) (layer "F.Cu") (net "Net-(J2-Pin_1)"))
 (segment (start 115.88 73.88) (end 115.88 74.5) (width 0.2) (layer "F.Cu") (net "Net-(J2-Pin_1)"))
 (segment (start 126.88 73.38) (end 125.5 72) (width 0.2) (layer "F.Cu") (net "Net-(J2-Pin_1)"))
 (segment (start 126.88 74.5) (end 126.88 73.38) (width 0.2) (layer "F.Cu") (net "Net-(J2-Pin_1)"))
 (segment (start 114 72) (end 125.5 72) (width 0.2) (layer "F.Cu") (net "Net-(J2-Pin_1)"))
 (segment (start 148.46 74.5) (end 148.46 83.89) (width 0.2) (layer "F.Cu") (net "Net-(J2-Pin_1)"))
 (segment (start 110.5 75.5) (end 110.5 73) (width 0.2) (layer "F.Cu") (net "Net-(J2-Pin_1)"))
 (segment (start 147 72) (end 148.46 73.46) (width 0.2) (layer "F.Cu") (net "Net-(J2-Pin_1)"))
 (segment (start 110.5 73) (end 111.5 72) (width 0.2) (layer "F.Cu") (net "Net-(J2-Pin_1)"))
 (segment (start 137.88 73.38) (end 136.5 72) (width 0.2) (layer "F.Cu") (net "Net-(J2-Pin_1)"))
 (segment (start 111.5 72) (end 114 72) (width 0.2) (layer "F.Cu") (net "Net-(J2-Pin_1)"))
 (segment (start 137.88 74.5) (end 137.88 73.38) (width 0.2) (layer "F.Cu") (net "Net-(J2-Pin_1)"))
 (segment (start 136.5 72) (end 147 72) (width 0.2) (layer "F.Cu") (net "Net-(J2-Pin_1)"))
 (segment (start 107.5 80.5) (end 107.5 78.5) (width 0.2) (layer "F.Cu") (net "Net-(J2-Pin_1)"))
 (segment (start 107.5 78.5) (end 110.5 75.5) (width 0.2) (layer "F.Cu") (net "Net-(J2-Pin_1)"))
 (via (at 112.5 85.5) (size 0.6) (drill 0.3) (layers "F.Cu" "B.Cu") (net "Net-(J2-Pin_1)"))
 (segment (start 119.5 88.42) (end 126.5 88.42) (width 0.2) (layer "B.Cu") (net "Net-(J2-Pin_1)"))
 (segment (start 115.42 88.42) (end 119.5 88.42) (width 0.2) (layer "B.Cu") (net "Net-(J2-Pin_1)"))
 (segment (start 140.5 88.42) (end 133.5 88.42) (width 0.2) (layer "B.Cu") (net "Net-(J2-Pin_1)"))
 (segment (start 133.5 88.42) (end 126.5 88.42) (width 0.2) (layer "B.Cu") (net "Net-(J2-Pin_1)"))
 (segment (start 112.5 85.5) (end 115.42 88.42) (width 0.2) (layer "B.Cu") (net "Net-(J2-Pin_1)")))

